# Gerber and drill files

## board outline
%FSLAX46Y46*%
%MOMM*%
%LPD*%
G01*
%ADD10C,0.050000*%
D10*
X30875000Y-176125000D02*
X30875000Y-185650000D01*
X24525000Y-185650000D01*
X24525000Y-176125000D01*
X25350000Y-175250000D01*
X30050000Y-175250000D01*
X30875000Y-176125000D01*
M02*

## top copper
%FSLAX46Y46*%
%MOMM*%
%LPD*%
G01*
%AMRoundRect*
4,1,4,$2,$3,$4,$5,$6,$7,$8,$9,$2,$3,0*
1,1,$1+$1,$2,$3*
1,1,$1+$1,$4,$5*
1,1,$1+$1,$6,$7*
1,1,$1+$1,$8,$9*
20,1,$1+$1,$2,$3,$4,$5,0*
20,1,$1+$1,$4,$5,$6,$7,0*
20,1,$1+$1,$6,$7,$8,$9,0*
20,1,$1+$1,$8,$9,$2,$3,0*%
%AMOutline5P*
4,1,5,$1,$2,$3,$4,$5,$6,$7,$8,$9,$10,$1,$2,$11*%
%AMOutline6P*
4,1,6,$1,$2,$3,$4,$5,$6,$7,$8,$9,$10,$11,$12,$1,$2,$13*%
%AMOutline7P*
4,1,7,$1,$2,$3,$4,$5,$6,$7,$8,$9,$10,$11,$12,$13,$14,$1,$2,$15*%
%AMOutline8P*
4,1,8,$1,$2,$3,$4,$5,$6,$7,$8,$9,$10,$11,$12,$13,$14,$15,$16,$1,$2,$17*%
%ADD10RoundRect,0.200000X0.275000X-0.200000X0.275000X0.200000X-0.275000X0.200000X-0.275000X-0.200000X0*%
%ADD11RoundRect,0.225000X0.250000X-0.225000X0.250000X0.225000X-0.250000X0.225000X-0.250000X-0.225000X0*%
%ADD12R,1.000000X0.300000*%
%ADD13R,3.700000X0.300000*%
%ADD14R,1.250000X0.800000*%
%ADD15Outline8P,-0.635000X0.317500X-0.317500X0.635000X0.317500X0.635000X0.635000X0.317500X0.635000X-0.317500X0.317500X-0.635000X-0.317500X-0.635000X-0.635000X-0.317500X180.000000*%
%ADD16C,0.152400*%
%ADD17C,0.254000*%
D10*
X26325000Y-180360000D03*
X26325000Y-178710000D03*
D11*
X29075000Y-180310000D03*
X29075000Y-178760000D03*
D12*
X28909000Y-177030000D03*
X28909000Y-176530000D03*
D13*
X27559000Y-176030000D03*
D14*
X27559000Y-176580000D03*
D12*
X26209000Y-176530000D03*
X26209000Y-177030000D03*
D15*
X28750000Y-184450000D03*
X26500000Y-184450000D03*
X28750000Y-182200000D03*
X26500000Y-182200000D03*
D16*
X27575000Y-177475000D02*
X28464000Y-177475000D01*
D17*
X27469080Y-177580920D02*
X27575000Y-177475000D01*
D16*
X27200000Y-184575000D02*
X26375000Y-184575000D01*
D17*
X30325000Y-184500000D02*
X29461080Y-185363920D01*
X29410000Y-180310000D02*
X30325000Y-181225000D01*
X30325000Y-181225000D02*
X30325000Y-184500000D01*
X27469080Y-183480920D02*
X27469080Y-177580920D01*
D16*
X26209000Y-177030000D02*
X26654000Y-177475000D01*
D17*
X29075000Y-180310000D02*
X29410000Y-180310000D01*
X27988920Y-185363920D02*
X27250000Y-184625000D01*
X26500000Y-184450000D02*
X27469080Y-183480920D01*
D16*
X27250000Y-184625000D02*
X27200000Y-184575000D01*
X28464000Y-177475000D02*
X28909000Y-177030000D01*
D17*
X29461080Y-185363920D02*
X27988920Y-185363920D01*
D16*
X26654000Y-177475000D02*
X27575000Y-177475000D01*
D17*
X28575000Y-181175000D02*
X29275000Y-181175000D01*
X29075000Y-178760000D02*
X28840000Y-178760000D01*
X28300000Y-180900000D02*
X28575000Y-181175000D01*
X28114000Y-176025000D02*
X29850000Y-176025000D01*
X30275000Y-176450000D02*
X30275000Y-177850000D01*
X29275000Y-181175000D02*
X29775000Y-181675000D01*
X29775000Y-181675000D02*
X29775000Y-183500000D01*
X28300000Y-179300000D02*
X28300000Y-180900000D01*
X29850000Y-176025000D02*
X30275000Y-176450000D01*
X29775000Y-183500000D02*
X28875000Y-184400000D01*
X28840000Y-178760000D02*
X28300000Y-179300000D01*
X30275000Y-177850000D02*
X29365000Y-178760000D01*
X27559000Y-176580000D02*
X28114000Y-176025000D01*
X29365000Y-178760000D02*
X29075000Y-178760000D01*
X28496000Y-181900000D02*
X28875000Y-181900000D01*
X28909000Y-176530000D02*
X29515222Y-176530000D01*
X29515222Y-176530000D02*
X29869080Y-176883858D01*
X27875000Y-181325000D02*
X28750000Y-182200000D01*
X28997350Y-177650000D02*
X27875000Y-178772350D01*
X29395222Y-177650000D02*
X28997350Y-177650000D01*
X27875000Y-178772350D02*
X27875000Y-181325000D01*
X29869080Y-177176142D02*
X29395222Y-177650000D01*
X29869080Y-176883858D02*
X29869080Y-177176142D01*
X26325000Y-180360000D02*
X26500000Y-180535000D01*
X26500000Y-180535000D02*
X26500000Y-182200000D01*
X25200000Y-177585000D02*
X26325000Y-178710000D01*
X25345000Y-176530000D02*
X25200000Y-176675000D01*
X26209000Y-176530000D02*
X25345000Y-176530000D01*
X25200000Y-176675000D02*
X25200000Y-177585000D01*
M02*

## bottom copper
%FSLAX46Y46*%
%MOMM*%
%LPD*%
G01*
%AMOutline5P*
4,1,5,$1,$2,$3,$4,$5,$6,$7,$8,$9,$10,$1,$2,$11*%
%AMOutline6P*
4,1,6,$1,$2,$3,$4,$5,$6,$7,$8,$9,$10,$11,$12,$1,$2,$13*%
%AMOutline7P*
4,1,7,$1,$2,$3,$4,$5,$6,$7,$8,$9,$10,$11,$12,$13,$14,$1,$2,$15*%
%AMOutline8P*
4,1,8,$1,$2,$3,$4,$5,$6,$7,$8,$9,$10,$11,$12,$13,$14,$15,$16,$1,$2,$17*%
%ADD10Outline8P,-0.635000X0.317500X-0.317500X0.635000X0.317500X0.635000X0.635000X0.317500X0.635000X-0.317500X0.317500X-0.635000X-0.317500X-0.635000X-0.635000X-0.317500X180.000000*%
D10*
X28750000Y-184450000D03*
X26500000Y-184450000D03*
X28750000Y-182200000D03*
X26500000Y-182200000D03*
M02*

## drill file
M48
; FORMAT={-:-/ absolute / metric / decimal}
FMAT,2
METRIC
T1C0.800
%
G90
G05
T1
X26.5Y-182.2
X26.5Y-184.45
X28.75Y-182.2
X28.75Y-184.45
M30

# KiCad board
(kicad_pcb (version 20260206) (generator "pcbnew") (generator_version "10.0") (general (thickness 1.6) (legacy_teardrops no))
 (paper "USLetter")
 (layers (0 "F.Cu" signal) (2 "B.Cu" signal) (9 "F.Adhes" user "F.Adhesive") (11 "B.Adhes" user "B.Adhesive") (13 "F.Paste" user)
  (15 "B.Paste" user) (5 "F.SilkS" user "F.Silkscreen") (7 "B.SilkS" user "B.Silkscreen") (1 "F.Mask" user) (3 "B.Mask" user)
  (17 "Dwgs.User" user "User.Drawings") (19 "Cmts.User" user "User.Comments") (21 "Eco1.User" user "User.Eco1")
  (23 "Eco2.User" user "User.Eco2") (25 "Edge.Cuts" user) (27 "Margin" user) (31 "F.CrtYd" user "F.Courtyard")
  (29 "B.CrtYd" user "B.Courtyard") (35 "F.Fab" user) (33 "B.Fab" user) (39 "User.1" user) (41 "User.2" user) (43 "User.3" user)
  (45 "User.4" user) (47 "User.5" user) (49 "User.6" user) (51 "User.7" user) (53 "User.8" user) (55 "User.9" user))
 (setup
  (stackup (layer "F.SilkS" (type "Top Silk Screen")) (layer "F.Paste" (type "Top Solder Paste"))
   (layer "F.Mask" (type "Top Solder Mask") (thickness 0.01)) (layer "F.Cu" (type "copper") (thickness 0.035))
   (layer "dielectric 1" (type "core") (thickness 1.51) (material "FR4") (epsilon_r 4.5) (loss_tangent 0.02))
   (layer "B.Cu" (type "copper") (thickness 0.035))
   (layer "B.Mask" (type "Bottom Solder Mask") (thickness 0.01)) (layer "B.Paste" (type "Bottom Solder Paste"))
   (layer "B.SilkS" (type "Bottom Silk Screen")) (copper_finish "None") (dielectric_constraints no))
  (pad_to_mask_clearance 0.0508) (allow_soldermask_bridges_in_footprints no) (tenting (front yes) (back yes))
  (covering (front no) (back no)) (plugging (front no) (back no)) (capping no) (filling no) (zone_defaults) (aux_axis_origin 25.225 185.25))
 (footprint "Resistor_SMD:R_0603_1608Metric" (layer "F.Cu") (at 26.325 179.535 90)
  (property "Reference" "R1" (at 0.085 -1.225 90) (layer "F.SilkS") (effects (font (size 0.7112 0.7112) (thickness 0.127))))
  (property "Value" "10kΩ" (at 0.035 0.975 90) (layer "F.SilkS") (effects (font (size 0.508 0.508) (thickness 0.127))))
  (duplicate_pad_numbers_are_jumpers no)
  (pad "1" smd roundrect (at -0.825 0 90) (size 0.8 0.95) (layers "F.Cu" "F.Mask" "F.Paste") (roundrect_rratio 0.25)
   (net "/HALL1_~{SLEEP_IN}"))
  (pad "2" smd roundrect (at 0.825 0 90) (size 0.8 0.95) (layers "F.Cu" "F.Mask" "F.Paste") (roundrect_rratio 0.25) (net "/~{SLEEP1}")))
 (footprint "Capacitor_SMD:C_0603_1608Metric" (layer "F.Cu") (at 29.075 179.535 90)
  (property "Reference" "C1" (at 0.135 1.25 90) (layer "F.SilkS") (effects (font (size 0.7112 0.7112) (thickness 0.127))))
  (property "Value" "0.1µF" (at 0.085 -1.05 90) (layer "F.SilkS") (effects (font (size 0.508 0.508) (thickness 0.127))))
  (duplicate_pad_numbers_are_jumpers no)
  (pad "1" smd roundrect (at -0.775 0 90) (size 0.9 0.95) (layers "F.Cu" "F.Mask" "F.Paste") (roundrect_rratio 0.25) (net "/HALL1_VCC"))
  (pad "2" smd roundrect (at 0.775 0 90) (size 0.9 0.95) (layers "F.Cu" "F.Mask" "F.Paste") (roundrect_rratio 0.25) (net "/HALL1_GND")))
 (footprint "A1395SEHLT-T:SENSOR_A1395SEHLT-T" (layer "F.Cu") (at 27.559 176.53 180)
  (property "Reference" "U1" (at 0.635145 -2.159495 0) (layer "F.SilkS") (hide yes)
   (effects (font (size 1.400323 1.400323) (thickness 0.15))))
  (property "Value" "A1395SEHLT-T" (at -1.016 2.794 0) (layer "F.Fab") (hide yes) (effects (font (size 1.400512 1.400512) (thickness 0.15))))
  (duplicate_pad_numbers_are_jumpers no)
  (pad "1" smd rect (at -1.35 -0.5 180) (size 1 0.3) (layers "F.Cu" "F.Mask" "F.Paste") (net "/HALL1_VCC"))
  (pad "2" smd rect (at -1.35 0 180) (size 1 0.3) (layers "F.Cu" "F.Mask" "F.Paste") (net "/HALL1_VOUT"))
  (pad "3" smd rect (at 0 0.5 90) (size 0.3 3.7) (layers "F.Cu" "F.Mask" "F.Paste") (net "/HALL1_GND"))
  (pad "4" smd rect (at 0 -0.05 180) (size 1.25 0.8) (layers "F.Cu" "F.Mask") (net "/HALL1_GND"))
  (pad "5" smd rect (at 1.35 0 180) (size 1 0.3) (layers "F.Cu" "F.Mask" "F.Paste") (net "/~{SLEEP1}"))
  (pad "6" smd rect (at 1.35 -0.5 180) (size 1 0.3) (layers "F.Cu" "F.Mask" "F.Paste") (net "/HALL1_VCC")))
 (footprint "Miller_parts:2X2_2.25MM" (layer "F.Cu") (at 27.625 183.325 180)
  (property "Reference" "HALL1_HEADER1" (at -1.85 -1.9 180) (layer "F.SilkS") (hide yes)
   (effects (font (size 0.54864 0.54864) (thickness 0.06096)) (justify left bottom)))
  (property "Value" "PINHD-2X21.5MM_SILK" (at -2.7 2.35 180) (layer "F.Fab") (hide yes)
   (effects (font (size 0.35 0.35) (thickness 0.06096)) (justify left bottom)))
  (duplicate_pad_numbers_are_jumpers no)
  (pad "P$1" thru_hole roundrect (at -1.125 -1.125 180) (size 1.27 1.27) (drill 0.8) (layers "*.Cu" "*.Mask") (remove_unused_layers no)
   (roundrect_rratio 0.25) (chamfer_ratio 0.25) (chamfer top_left top_right bottom_left bottom_right) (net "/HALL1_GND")
   (solder_mask_margin 0.0762))
  (pad "P$2" thru_hole roundrect (at 1.125 -1.125 180) (size 1.27 1.27) (drill 0.8) (layers "*.Cu" "*.Mask") (remove_unused_layers no)
   (roundrect_rratio 0.25) (chamfer_ratio 0.25) (chamfer top_left top_right bottom_left bottom_right) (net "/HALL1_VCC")
   (solder_mask_margin 0.0762))
  (pad "P$3" thru_hole roundrect (at -1.125 1.125 180) (size 1.27 1.27) (drill 0.8) (layers "*.Cu" "*.Mask") (remove_unused_layers no)
   (roundrect_rratio 0.25) (chamfer_ratio 0.25) (chamfer top_left top_right bottom_left bottom_right) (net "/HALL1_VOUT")
   (solder_mask_margin 0.0762))
  (pad "P$4" thru_hole roundrect (at 1.125 1.125 180) (size 1.27 1.27) (drill 0.8) (layers "*.Cu" "*.Mask") (remove_unused_layers no)
   (roundrect_rratio 0.25) (chamfer_ratio 0.25) (chamfer top_left top_right bottom_left bottom_right) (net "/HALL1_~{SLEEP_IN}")
   (solder_mask_margin 0.0762)))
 (gr_poly
  (pts (xy 30.875 176.125) (xy 30.875 185.65) (xy 24.525 185.65) (xy 24.525 176.125) (xy 25.35 175.25) (xy 30.05 175.25))
  (stroke (width 0.05) (type solid)) (fill no) (layer "Edge.Cuts"))
 (segment (start 27.575 177.475) (end 28.464 177.475) (width 0.1524) (layer "F.Cu") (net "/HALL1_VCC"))
 (segment (start 27.46908 177.58092) (end 27.575 177.475) (width 0.254) (layer "F.Cu") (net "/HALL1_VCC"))
 (segment (start 27.2 184.575) (end 26.375 184.575) (width 0.1524) (layer "F.Cu") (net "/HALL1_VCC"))
 (segment (start 30.325 184.5) (end 29.46108 185.36392) (width 0.254) (layer "F.Cu") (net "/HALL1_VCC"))
 (segment (start 29.41 180.31) (end 30.325 181.225) (width 0.254) (layer "F.Cu") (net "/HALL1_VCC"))
 (segment (start 30.325 181.225) (end 30.325 184.5) (width 0.254) (layer "F.Cu") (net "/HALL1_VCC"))
 (segment (start 27.46908 183.48092) (end 27.46908 177.58092) (width 0.254) (layer "F.Cu") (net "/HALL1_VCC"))
 (segment (start 26.209 177.03) (end 26.654 177.475) (width 0.1524) (layer "F.Cu") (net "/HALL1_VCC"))
 (segment (start 29.075 180.31) (end 29.41 180.31) (width 0.254) (layer "F.Cu") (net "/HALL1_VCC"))
 (segment (start 27.98892 185.36392) (end 27.25 184.625) (width 0.254) (layer "F.Cu") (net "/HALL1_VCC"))
 (segment (start 26.5 184.45) (end 27.46908 183.48092) (width 0.254) (layer "F.Cu") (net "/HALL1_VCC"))
 (segment (start 27.25 184.625) (end 27.2 184.575) (width 0.1524) (layer "F.Cu") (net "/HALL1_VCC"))
 (segment (start 28.464 177.475) (end 28.909 177.03) (width 0.1524) (layer "F.Cu") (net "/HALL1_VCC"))
 (segment (start 29.46108 185.36392) (end 27.98892 185.36392) (width 0.254) (layer "F.Cu") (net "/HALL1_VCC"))
 (segment (start 26.654 177.475) (end 27.575 177.475) (width 0.1524) (layer "F.Cu") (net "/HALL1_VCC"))
 (segment (start 28.575 181.175) (end 29.275 181.175) (width 0.254) (layer "F.Cu") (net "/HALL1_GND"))
 (segment (start 29.075 178.76) (end 28.84 178.76) (width 0.254) (layer "F.Cu") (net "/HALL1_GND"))
 (segment (start 28.3 180.9) (end 28.575 181.175) (width 0.254) (layer "F.Cu") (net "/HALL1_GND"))
 (segment (start 28.114 176.025) (end 29.85 176.025) (width 0.254) (layer "F.Cu") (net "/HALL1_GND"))
 (segment (start 30.275 176.45) (end 30.275 177.85) (width 0.254) (layer "F.Cu") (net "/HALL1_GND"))
 (segment (start 29.275 181.175) (end 29.775 181.675) (width 0.254) (layer "F.Cu") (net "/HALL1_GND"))
 (segment (start 29.775 181.675) (end 29.775 183.5) (width 0.254) (layer "F.Cu") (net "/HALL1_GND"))
 (segment (start 28.3 179.3) (end 28.3 180.9) (width 0.254) (layer "F.Cu") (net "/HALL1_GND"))
 (segment (start 29.85 176.025) (end 30.275 176.45) (width 0.254) (layer "F.Cu") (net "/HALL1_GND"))
 (segment (start 29.775 183.5) (end 28.875 184.4) (width 0.254) (layer "F.Cu") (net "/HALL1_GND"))
 (segment (start 28.84 178.76) (end 28.3 179.3) (width 0.254) (layer "F.Cu") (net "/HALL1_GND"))
 (segment (start 30.275 177.85) (end 29.365 178.76) (width 0.254) (layer "F.Cu") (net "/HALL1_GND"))
 (segment (start 27.559 176.58) (end 28.114 176.025) (width 0.254) (layer "F.Cu") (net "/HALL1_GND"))
 (segment (start 29.365 178.76) (end 29.075 178.76) (width 0.254) (layer "F.Cu") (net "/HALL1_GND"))
 (segment (start 28.496 181.9) (end 28.875 181.9) (width 0.254) (layer "F.Cu") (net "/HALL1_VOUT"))
 (segment (start 28.909 176.53) (end 29.515222 176.53) (width 0.254) (layer "F.Cu") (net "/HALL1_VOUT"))
 (segment (start 29.515222 176.53) (end 29.86908 176.883858) (width 0.254) (layer "F.Cu") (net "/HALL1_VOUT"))
 (segment (start 27.875 181.325) (end 28.75 182.2) (width 0.254) (layer "F.Cu") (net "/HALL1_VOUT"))
 (segment (start 28.99735 177.65) (end 27.875 178.77235) (width 0.254) (layer "F.Cu") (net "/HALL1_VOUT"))
 (segment (start 29.395222 177.65) (end 28.99735 177.65) (width 0.254) (layer "F.Cu") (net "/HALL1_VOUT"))
 (segment (start 27.875 178.77235) (end 27.875 181.325) (width 0.254) (layer "F.Cu") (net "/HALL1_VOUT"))
 (segment (start 29.86908 177.176142) (end 29.395222 177.65) (width 0.254) (layer "F.Cu") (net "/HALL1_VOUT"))
 (segment (start 29.86908 176.883858) (end 29.86908 177.176142) (width 0.254) (layer "F.Cu") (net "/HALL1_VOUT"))
 (segment (start 26.325 180.36) (end 26.5 180.535) (width 0.254) (layer "F.Cu") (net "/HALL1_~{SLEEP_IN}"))
 (segment (start 26.5 180.535) (end 26.5 182.2) (width 0.254) (layer "F.Cu") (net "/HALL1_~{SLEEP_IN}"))
 (segment (start 25.2 177.585) (end 26.325 178.71) (width 0.254) (layer "F.Cu") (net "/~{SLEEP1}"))
 (segment (start 25.345 176.53) (end 25.2 176.675) (width 0.254) (layer "F.Cu") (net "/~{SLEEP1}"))
 (segment (start 26.209 176.53) (end 25.345 176.53) (width 0.254) (layer "F.Cu") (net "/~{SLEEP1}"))
 (segment (start 25.2 176.675) (end 25.2 177.585) (width 0.254) (layer "F.Cu") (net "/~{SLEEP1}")))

